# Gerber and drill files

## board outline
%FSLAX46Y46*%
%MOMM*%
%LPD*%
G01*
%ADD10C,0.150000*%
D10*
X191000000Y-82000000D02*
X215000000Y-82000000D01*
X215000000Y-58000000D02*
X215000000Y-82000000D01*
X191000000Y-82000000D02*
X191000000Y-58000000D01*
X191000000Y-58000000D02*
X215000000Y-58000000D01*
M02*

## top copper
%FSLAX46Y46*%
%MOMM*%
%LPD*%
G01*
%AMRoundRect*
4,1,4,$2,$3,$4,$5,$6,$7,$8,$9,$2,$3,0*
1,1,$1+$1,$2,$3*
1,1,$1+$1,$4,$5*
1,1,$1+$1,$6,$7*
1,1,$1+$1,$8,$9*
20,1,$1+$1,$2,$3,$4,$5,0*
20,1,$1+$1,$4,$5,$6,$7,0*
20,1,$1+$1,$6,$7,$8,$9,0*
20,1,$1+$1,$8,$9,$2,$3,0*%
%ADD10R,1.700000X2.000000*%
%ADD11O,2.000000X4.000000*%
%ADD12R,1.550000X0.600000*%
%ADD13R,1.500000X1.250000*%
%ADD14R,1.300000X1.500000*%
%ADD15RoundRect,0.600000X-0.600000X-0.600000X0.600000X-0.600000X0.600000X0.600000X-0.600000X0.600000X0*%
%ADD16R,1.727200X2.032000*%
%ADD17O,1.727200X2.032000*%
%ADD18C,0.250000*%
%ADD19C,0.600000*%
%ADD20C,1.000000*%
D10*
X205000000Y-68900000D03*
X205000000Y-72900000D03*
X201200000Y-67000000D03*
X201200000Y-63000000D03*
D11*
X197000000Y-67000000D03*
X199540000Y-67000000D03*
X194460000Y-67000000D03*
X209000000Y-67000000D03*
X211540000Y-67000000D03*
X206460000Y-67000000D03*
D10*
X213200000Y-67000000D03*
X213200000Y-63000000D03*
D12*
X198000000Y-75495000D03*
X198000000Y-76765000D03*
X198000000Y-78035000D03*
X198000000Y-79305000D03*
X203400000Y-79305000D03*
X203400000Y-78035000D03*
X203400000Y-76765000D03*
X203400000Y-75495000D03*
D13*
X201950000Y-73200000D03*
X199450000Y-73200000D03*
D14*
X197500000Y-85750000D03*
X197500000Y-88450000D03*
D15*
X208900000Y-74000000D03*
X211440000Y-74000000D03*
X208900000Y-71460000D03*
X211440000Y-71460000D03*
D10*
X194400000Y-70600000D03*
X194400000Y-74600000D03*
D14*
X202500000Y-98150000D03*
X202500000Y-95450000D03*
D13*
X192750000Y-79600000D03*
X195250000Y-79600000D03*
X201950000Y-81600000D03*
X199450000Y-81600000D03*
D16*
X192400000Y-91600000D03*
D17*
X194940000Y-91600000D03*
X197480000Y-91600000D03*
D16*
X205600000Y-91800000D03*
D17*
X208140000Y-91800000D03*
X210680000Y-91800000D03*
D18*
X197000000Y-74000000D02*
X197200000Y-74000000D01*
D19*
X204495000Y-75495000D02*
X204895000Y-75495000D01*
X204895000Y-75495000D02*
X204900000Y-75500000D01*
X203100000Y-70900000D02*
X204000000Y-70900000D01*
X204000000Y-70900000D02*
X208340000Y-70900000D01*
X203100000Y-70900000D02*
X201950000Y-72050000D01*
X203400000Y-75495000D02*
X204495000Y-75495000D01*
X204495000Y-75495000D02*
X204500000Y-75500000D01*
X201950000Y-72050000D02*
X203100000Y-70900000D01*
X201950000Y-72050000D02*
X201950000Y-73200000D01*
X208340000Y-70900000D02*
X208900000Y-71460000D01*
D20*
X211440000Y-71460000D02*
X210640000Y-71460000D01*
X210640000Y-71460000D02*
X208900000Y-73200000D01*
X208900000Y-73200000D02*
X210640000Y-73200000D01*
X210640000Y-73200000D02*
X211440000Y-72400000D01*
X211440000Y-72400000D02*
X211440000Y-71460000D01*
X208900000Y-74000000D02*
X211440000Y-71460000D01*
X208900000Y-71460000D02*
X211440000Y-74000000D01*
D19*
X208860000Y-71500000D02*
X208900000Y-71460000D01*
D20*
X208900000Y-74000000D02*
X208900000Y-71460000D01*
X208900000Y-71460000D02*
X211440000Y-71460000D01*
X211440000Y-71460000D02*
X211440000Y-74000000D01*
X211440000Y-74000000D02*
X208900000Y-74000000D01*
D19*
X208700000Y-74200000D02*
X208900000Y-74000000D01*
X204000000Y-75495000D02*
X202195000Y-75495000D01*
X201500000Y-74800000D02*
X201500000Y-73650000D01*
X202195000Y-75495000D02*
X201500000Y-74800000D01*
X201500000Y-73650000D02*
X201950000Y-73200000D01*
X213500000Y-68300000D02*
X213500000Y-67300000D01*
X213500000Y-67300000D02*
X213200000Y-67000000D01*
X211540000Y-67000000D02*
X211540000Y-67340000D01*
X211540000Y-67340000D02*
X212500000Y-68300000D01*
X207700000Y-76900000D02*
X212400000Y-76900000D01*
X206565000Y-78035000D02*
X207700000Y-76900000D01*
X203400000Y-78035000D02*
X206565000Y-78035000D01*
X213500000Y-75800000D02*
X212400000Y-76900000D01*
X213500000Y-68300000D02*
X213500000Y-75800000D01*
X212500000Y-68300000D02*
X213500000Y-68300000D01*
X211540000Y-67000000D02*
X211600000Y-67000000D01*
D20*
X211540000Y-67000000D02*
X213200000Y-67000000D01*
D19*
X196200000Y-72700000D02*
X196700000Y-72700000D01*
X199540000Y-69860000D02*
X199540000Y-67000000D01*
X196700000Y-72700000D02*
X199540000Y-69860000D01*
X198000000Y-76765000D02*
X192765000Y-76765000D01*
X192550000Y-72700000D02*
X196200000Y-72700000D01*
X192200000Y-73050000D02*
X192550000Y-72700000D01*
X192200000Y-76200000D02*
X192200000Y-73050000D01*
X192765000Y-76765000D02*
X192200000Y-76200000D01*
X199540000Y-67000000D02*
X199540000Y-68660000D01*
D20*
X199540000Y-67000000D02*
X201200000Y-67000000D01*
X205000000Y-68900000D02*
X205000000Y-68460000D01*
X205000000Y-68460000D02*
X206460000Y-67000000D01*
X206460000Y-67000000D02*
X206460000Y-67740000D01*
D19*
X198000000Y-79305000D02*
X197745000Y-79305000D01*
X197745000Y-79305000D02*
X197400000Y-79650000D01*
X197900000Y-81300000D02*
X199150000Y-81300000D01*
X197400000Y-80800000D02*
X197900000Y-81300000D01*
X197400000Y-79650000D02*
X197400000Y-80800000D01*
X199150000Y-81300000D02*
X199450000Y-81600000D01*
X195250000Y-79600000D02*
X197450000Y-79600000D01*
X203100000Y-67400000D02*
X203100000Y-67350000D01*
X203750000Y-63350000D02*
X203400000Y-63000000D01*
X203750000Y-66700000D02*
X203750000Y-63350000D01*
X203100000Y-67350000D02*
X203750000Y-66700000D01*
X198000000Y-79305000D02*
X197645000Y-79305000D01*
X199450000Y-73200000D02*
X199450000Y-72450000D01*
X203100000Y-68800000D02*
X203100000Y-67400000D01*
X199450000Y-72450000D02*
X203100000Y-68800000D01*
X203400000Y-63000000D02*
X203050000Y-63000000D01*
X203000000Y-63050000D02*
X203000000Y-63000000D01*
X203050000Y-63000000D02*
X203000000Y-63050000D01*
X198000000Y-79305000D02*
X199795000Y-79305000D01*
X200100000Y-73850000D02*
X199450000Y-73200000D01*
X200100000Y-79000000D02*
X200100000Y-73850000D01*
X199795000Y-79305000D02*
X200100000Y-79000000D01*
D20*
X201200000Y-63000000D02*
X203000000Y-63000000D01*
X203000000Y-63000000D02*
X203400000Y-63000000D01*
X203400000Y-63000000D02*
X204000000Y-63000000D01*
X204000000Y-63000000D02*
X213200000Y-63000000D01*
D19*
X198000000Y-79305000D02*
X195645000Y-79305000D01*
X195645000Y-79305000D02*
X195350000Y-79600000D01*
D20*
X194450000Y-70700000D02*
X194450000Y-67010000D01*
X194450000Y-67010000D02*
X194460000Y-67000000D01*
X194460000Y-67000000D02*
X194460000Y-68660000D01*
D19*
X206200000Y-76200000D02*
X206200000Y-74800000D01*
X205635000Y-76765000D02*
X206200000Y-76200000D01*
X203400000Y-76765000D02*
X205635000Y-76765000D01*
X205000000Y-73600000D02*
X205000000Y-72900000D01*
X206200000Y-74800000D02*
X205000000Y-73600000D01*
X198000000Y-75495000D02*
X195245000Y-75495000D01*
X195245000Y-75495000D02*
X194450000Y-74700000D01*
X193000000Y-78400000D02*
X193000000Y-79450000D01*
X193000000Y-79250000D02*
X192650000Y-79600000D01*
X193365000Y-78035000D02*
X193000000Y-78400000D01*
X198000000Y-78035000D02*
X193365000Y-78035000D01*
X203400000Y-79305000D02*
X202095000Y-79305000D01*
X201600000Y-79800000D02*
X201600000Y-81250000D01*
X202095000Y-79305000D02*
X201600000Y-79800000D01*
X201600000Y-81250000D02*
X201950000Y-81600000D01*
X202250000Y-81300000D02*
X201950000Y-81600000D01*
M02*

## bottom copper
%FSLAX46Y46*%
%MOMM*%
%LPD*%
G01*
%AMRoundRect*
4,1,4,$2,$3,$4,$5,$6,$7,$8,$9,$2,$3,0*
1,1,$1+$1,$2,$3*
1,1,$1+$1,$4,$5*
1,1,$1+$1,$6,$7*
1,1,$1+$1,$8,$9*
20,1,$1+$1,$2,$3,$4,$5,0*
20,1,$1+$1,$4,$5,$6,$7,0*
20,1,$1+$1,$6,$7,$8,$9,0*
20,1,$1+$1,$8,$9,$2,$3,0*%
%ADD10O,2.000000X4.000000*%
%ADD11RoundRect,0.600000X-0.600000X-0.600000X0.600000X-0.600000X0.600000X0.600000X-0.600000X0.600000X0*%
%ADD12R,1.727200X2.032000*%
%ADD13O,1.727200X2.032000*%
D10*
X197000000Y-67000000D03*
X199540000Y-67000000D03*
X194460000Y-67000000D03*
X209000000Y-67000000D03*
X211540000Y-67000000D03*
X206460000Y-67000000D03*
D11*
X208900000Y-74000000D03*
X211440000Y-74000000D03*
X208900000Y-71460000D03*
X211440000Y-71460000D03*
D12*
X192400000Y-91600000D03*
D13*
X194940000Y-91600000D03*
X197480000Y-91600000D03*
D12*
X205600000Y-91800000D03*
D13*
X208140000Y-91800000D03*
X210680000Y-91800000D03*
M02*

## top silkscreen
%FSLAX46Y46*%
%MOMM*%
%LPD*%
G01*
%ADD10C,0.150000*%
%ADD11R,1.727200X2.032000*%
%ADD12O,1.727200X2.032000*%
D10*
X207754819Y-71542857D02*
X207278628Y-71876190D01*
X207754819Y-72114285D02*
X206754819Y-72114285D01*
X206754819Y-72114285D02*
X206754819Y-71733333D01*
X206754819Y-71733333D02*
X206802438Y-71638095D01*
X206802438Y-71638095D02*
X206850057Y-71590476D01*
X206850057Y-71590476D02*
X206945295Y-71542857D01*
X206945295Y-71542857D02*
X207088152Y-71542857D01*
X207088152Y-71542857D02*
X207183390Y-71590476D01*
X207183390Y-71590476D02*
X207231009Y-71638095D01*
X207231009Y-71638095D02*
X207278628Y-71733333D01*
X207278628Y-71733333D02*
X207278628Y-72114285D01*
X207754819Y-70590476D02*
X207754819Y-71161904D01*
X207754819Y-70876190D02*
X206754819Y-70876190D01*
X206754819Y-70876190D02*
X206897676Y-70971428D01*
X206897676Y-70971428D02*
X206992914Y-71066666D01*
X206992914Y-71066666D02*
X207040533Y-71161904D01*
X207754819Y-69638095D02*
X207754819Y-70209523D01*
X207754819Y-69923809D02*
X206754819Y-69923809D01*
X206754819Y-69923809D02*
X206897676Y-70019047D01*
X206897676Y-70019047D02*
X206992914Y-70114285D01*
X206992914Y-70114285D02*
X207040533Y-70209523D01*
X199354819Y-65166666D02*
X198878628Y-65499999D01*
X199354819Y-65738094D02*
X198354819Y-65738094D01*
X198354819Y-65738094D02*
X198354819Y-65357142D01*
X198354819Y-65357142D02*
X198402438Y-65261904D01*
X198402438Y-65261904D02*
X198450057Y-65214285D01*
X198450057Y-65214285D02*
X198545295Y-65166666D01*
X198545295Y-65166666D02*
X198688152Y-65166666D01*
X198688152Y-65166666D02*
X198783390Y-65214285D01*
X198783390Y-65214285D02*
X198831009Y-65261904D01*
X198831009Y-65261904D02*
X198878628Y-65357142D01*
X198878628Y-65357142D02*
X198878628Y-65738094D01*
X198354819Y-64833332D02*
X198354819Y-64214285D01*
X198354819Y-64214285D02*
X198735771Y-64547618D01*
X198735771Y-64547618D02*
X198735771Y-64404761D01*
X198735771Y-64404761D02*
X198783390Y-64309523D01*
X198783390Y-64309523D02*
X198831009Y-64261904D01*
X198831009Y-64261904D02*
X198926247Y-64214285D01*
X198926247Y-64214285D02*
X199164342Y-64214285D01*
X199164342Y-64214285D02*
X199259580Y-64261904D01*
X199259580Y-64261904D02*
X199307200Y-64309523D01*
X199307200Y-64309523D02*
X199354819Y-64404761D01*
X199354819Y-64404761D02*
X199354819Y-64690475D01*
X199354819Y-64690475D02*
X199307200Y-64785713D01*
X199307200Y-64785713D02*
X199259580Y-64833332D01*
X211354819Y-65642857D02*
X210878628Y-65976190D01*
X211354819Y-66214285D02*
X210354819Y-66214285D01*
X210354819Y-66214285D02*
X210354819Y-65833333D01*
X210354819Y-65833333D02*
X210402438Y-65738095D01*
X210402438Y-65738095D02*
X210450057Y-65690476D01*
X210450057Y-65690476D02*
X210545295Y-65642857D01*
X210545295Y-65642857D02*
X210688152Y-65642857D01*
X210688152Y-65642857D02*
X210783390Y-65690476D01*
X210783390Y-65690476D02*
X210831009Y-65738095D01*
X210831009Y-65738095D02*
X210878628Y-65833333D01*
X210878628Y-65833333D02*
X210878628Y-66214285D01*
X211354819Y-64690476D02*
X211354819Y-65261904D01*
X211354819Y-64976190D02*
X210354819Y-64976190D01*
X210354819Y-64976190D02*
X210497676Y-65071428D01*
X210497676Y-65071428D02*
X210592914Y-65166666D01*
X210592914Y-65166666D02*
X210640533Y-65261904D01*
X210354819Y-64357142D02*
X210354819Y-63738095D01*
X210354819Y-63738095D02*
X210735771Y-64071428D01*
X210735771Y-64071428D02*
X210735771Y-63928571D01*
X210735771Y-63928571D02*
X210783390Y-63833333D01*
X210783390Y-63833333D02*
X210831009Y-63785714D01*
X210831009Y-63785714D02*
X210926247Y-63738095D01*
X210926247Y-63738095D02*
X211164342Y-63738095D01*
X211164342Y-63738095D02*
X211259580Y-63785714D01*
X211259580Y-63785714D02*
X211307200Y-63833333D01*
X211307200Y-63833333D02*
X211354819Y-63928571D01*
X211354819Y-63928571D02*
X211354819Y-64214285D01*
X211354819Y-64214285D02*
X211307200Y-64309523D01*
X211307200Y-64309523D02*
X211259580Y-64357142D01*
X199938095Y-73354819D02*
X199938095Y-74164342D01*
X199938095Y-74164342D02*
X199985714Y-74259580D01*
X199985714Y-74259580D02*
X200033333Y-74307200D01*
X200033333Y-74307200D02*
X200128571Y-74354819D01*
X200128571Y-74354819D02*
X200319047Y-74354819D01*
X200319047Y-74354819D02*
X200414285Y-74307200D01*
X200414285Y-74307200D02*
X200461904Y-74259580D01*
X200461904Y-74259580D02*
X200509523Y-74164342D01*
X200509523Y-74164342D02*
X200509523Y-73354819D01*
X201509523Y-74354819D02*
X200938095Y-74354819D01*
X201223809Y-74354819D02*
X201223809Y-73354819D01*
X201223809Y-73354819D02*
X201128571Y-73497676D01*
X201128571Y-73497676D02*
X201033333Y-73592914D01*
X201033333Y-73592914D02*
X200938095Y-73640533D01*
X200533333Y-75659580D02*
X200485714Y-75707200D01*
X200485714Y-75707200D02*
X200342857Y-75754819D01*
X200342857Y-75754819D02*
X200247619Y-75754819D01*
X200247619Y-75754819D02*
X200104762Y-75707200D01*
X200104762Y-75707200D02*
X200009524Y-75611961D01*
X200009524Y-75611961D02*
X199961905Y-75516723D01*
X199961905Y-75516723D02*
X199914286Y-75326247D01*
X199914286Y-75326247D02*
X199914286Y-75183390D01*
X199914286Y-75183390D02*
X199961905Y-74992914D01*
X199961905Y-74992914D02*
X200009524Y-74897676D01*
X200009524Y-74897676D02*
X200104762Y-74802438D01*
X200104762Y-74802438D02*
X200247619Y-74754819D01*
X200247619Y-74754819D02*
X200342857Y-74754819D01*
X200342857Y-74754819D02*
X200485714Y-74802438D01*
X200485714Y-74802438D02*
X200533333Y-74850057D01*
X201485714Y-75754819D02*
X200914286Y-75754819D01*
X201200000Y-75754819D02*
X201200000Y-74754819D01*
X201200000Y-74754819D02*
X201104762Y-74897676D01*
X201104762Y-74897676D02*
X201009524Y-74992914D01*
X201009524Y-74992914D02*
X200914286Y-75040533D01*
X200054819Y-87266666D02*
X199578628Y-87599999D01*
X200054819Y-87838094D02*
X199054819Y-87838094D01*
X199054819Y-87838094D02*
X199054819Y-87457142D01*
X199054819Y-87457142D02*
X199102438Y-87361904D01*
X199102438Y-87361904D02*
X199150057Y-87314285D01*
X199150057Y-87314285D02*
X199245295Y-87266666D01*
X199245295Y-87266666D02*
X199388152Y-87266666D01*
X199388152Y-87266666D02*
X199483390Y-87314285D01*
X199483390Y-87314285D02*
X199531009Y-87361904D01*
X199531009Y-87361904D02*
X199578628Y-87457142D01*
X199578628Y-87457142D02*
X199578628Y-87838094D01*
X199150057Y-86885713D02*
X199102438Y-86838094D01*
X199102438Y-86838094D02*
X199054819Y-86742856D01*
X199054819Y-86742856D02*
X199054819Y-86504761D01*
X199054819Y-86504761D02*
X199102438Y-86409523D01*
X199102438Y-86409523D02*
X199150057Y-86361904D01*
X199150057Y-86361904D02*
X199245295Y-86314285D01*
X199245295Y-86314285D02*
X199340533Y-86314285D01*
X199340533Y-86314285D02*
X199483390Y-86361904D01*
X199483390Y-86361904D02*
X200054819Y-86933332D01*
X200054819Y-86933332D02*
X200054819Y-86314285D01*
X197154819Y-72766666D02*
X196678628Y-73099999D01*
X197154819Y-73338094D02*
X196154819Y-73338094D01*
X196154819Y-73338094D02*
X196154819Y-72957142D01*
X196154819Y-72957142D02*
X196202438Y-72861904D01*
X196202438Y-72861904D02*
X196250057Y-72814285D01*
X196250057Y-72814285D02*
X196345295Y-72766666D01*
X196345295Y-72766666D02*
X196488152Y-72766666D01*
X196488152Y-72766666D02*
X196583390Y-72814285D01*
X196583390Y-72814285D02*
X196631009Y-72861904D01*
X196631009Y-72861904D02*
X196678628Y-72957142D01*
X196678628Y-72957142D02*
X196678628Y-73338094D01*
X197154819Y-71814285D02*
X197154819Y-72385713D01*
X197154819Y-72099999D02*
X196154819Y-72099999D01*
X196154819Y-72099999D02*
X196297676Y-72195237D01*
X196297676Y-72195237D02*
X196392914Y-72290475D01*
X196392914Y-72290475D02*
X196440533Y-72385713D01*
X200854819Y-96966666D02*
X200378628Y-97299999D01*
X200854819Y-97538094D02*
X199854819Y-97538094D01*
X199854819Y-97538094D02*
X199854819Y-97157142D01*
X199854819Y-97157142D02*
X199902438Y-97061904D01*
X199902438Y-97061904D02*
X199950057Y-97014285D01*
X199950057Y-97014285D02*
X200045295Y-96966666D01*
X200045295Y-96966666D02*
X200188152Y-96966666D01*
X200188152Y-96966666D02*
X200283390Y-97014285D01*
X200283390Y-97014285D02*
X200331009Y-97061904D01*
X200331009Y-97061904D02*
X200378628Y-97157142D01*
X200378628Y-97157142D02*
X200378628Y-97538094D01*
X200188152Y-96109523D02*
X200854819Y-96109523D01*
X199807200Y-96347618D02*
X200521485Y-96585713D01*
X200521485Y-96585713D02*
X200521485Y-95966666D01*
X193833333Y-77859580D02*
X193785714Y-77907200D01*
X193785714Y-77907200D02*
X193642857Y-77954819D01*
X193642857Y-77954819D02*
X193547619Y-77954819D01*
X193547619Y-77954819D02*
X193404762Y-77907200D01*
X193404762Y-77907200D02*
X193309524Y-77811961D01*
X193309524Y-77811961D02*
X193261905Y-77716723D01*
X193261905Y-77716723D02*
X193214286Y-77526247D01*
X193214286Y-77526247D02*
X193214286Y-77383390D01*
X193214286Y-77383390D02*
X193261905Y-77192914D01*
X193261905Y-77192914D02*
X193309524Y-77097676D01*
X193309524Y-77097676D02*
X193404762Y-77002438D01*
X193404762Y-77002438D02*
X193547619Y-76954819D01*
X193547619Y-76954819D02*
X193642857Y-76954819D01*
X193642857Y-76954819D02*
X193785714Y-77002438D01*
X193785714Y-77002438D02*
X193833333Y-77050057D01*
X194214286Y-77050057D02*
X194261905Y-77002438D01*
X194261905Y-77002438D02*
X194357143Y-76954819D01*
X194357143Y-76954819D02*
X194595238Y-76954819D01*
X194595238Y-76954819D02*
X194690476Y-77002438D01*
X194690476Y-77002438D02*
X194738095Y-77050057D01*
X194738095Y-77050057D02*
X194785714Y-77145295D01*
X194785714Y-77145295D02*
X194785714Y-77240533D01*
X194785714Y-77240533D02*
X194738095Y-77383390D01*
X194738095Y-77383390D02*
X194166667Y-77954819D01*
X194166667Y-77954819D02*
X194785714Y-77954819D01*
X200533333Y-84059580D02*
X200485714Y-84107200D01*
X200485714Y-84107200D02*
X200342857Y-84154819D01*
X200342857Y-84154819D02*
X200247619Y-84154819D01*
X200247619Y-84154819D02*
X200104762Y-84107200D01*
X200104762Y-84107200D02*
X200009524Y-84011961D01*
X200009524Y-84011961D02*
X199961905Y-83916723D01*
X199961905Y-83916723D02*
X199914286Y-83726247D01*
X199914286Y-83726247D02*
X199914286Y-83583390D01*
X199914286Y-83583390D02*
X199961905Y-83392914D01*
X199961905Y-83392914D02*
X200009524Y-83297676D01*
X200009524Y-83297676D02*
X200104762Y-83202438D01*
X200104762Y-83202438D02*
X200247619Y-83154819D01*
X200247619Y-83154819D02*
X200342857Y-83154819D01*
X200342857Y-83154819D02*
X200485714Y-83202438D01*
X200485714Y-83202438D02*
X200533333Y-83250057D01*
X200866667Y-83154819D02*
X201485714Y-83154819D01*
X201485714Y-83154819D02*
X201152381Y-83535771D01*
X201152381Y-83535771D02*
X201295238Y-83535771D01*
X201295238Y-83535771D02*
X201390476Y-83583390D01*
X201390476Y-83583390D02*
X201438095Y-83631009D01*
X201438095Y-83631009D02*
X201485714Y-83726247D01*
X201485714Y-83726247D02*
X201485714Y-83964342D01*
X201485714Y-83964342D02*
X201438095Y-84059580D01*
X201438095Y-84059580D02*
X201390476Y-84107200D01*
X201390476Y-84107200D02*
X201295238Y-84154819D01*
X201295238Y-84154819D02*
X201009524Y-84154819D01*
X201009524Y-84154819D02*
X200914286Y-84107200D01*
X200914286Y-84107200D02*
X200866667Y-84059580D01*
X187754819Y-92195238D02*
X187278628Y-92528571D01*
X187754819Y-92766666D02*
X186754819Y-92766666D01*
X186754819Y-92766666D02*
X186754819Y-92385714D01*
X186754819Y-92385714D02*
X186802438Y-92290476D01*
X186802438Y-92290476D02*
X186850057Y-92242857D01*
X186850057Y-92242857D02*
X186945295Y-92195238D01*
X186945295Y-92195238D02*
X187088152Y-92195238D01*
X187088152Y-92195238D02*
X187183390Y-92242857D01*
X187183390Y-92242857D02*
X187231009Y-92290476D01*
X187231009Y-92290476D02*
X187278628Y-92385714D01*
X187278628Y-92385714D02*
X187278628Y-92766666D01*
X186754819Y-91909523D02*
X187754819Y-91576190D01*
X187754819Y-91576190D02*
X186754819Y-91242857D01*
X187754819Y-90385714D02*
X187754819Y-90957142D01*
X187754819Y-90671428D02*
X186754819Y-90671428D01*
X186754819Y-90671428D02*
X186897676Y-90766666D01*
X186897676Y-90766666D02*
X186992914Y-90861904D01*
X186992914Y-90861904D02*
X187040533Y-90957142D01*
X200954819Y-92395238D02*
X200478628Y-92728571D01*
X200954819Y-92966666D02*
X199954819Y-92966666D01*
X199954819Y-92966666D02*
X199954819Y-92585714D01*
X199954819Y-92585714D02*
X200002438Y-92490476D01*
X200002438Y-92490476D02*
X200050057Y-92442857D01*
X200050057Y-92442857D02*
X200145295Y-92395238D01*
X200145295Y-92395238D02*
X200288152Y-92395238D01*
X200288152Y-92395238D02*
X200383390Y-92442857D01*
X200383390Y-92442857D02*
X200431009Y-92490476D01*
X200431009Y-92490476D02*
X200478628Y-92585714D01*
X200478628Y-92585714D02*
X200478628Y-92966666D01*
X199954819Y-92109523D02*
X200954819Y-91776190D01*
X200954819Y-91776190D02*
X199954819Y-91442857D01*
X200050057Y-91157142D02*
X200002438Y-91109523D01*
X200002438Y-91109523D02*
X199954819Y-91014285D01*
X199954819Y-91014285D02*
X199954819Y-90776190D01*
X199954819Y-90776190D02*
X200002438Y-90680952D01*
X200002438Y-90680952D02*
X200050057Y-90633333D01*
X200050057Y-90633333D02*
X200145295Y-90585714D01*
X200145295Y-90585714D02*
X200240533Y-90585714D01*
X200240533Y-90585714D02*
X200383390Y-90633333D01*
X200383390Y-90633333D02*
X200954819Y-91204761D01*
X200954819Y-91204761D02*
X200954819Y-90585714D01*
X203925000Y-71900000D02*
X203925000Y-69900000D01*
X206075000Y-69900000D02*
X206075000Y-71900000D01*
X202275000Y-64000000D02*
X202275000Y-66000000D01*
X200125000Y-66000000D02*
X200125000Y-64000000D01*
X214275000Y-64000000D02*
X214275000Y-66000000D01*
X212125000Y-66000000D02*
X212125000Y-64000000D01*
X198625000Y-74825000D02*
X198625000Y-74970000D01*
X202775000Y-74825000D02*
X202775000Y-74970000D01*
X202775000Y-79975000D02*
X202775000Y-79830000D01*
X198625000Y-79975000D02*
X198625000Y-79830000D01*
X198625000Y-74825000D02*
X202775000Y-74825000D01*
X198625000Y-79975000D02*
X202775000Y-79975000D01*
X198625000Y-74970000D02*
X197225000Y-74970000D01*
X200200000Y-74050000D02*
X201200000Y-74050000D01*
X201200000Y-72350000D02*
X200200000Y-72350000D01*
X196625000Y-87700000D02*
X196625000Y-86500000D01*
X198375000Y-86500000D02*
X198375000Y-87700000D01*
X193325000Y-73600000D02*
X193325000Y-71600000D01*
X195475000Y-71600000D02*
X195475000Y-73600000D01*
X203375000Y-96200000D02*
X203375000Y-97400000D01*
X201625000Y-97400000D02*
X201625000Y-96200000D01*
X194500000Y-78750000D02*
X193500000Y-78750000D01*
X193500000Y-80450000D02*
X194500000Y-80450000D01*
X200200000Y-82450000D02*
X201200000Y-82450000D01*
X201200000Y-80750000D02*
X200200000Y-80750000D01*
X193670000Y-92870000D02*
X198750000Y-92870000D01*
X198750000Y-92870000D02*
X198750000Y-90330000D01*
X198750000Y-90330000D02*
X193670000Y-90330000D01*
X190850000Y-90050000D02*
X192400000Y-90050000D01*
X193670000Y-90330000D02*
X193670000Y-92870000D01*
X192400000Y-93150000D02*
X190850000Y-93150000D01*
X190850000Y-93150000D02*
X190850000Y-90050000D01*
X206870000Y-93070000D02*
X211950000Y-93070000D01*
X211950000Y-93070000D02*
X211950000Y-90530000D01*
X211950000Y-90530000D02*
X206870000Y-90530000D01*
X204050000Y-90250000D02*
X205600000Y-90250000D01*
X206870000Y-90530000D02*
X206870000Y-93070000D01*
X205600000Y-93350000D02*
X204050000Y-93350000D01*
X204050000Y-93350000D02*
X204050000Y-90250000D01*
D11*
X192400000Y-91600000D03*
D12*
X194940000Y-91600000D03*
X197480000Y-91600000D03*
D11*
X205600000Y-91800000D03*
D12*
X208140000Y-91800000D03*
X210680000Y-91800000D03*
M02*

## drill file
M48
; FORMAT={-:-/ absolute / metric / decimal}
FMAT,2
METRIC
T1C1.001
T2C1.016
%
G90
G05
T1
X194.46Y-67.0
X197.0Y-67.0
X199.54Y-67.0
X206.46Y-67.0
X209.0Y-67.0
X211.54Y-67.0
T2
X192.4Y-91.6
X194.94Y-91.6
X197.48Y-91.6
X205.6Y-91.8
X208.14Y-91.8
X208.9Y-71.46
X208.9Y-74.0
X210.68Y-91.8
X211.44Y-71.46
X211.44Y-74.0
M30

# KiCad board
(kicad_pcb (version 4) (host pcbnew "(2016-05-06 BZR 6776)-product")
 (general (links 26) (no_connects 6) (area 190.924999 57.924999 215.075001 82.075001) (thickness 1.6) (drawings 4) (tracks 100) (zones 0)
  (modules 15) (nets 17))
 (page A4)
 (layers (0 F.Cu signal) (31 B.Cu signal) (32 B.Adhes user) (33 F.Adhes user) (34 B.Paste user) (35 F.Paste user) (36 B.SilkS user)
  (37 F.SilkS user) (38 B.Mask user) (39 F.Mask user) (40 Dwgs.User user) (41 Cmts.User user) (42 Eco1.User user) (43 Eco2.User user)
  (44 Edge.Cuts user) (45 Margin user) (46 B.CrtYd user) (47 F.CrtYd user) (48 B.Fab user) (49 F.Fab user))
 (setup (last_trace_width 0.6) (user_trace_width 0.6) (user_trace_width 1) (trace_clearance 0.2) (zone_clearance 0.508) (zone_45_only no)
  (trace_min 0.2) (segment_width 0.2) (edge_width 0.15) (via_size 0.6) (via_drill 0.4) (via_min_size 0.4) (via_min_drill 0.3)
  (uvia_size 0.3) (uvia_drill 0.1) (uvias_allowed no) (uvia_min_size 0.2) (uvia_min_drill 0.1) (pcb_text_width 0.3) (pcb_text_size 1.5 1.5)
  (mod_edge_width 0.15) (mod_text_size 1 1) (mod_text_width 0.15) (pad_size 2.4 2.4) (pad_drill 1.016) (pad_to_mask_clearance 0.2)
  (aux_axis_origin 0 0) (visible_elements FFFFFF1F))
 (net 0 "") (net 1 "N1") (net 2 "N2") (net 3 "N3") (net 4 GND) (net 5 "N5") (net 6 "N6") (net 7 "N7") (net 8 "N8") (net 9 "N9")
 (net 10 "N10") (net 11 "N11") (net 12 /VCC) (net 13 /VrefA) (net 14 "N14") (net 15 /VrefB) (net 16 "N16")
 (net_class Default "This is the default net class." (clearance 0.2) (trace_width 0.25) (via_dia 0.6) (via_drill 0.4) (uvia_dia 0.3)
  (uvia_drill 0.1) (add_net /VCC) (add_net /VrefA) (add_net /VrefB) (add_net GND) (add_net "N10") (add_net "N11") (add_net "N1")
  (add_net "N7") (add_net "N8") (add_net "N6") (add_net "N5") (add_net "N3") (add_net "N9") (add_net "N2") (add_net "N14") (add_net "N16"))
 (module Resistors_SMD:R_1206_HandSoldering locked (layer F.Cu) (at 205 70.9 270)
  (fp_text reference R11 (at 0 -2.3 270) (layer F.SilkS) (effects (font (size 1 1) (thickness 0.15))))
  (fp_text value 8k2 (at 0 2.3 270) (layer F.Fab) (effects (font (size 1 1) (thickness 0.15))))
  (fp_line (start 1 1.075) (end -1 1.075) (layer F.SilkS) (width 0.15))
  (fp_line (start -1 -1.075) (end 1 -1.075) (layer F.SilkS) (width 0.15))
  (pad 1 smd rect (at -2 0 270) (size 2 1.7) (layers F.Cu F.Paste F.Mask) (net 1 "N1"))
  (pad 2 smd rect (at 2 0 270) (size 2 1.7) (layers F.Cu F.Paste F.Mask) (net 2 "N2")))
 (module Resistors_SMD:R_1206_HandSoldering (layer F.Cu) (at 201.2 65 90)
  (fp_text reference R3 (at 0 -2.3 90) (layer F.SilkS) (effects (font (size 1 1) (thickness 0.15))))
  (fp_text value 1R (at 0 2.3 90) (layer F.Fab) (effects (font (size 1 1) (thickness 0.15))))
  (fp_line (start 1 1.075) (end -1 1.075) (layer F.SilkS) (width 0.15))
  (fp_line (start -1 -1.075) (end 1 -1.075) (layer F.SilkS) (width 0.15))
  (pad 1 smd rect (at -2 0 90) (size 2 1.7) (layers F.Cu F.Paste F.Mask) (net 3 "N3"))
  (pad 2 smd rect (at 2 0 90) (size 2 1.7) (layers F.Cu F.Paste F.Mask) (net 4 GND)))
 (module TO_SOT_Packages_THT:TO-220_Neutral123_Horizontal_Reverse (layer B.Cu) (at 197 67 180)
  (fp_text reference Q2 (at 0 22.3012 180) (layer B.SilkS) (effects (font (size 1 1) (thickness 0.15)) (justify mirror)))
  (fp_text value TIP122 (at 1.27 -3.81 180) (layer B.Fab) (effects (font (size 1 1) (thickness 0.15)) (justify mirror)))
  (pad 2 thru_hole oval (at 0 0 90) (size 4 2) (drill 1.00076) (layers *.Cu *.Mask B.SilkS) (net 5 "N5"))
  (pad 3 thru_hole oval (at -2.54 0 90) (size 4 2) (drill 1.00076) (layers *.Cu *.Mask B.SilkS) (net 3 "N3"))
  (pad 1 thru_hole oval (at 2.54 0 90) (size 4 2) (drill 1.00076) (layers *.Cu *.Mask B.SilkS) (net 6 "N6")))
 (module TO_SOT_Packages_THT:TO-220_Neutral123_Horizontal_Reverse (layer B.Cu) (at 209 67 180)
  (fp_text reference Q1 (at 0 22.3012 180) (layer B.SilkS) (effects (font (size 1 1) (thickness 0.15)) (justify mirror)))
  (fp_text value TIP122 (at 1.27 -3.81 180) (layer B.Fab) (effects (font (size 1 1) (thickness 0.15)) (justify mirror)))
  (pad 2 thru_hole oval (at 0 0 90) (size 4 2) (drill 1.00076) (layers *.Cu *.Mask B.SilkS) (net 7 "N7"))
  (pad 3 thru_hole oval (at -2.54 0 90) (size 4 2) (drill 1.00076) (layers *.Cu *.Mask B.SilkS) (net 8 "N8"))
  (pad 1 thru_hole oval (at 2.54 0 90) (size 4 2) (drill 1.00076) (layers *.Cu *.Mask B.SilkS) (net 1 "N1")))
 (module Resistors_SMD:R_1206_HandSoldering (layer F.Cu) (at 213.2 65 90)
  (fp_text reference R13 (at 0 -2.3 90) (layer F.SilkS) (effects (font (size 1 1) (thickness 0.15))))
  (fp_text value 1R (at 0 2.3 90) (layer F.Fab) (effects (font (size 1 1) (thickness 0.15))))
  (fp_line (start 1 1.075) (end -1 1.075) (layer F.SilkS) (width 0.15))
  (fp_line (start -1 -1.075) (end 1 -1.075) (layer F.SilkS) (width 0.15))
  (pad 1 smd rect (at -2 0 90) (size 2 1.7) (layers F.Cu F.Paste F.Mask) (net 8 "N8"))
  (pad 2 smd rect (at 2 0 90) (size 2 1.7) (layers F.Cu F.Paste F.Mask) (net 4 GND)))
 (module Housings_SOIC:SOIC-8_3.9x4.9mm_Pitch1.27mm (layer F.Cu) (at 200.7 77.4)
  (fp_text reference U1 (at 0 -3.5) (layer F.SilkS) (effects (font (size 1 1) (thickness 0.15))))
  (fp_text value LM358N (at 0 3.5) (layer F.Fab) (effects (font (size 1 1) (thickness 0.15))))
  (fp_line (start -2.075 -2.575) (end -2.075 -2.43) (layer F.SilkS) (width 0.15))
  (fp_line (start 2.075 -2.575) (end 2.075 -2.43) (layer F.SilkS) (width 0.15))
  (fp_line (start 2.075 2.575) (end 2.075 2.43) (layer F.SilkS) (width 0.15))
  (fp_line (start -2.075 2.575) (end -2.075 2.43) (layer F.SilkS) (width 0.15))
  (fp_line (start -2.075 -2.575) (end 2.075 -2.575) (layer F.SilkS) (width 0.15))
  (fp_line (start -2.075 2.575) (end 2.075 2.575) (layer F.SilkS) (width 0.15))
  (fp_line (start -2.075 -2.43) (end -3.475 -2.43) (layer F.SilkS) (width 0.15))
  (pad 1 smd rect (at -2.7 -1.905) (size 1.55 0.6) (layers F.Cu F.Paste F.Mask) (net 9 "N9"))
  (pad 2 smd rect (at -2.7 -0.635) (size 1.55 0.6) (layers F.Cu F.Paste F.Mask) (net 3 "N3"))
  (pad 3 smd rect (at -2.7 0.635) (size 1.55 0.6) (layers F.Cu F.Paste F.Mask) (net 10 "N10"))
  (pad 4 smd rect (at -2.7 1.905) (size 1.55 0.6) (layers F.Cu F.Paste F.Mask) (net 4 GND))
  (pad 5 smd rect (at 2.7 1.905) (size 1.55 0.6) (layers F.Cu F.Paste F.Mask) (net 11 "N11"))
  (pad 6 smd rect (at 2.7 0.635) (size 1.55 0.6) (layers F.Cu F.Paste F.Mask) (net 8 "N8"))
  (pad 7 smd rect (at 2.7 -0.635) (size 1.55 0.6) (layers F.Cu F.Paste F.Mask) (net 2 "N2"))
  (pad 8 smd rect (at 2.7 -1.905) (size 1.55 0.6) (layers F.Cu F.Paste F.Mask) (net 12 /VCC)))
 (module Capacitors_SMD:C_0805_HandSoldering (layer F.Cu) (at 200.7 73.2 180)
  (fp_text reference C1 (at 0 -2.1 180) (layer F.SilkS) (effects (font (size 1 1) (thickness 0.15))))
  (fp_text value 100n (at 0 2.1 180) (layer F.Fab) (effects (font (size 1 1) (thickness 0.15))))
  (fp_line (start 0.5 -0.85) (end -0.5 -0.85) (layer F.SilkS) (width 0.15))
  (fp_line (start -0.5 0.85) (end 0.5 0.85) (layer F.SilkS) (width 0.15))
  (pad 1 smd rect (at -1.25 0 180) (size 1.5 1.25) (layers F.Cu F.Paste F.Mask) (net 12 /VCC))
  (pad 2 smd rect (at 1.25 0 180) (size 1.5 1.25) (layers F.Cu F.Paste F.Mask) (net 4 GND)))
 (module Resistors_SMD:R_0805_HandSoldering (layer F.Cu) (at 197.5 87.1 270)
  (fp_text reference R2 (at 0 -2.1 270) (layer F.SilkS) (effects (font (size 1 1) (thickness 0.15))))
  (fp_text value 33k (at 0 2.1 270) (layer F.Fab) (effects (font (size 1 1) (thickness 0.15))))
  (fp_line (start 0.6 0.875) (end -0.6 0.875) (layer F.SilkS) (width 0.15))
  (fp_line (start -0.6 -0.875) (end 0.6 -0.875) (layer F.SilkS) (width 0.15))
  (pad 1 smd rect (at -1.35 0 270) (size 1.5 1.3) (layers F.Cu F.Paste F.Mask) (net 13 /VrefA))
  (pad 2 smd rect (at 1.35 0 270) (size 1.5 1.3) (layers F.Cu F.Paste F.Mask) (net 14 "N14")))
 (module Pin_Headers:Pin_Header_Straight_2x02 (layer B.Cu) (at 208.9 74)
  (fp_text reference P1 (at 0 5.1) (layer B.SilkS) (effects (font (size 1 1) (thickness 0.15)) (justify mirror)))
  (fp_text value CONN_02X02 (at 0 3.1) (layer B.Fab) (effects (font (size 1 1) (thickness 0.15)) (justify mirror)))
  (pad 1 thru_hole roundrect (at 0 0) (size 2.4 2.4) (drill 1.016) (layers *.Cu *.Mask B.SilkS) (roundrect_rratio 0.25) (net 12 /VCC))
  (pad 2 thru_hole roundrect (at 2.54 0) (size 2.4 2.4) (drill 1.016) (layers *.Cu *.Mask B.SilkS) (roundrect_rratio 0.25) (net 12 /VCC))
  (pad 3 thru_hole roundrect (at 0 -2.54) (size 2.4 2.4) (drill 1.016) (layers *.Cu *.Mask B.SilkS) (roundrect_rratio 0.25) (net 12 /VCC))
  (pad 4 thru_hole roundrect (at 2.54 -2.54) (size 2.4 2.4) (drill 1.016) (layers *.Cu *.Mask B.SilkS) (roundrect_rratio 0.25) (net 12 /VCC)))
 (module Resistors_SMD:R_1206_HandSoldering (layer F.Cu) (at 194.4 72.6 270)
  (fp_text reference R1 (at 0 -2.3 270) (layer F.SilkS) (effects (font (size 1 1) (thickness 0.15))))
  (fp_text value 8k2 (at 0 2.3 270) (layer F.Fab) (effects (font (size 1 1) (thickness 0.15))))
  (fp_line (start 1 1.075) (end -1 1.075) (layer F.SilkS) (width 0.15))
  (fp_line (start -1 -1.075) (end 1 -1.075) (layer F.SilkS) (width 0.15))
  (pad 1 smd rect (at -2 0 270) (size 2 1.7) (layers F.Cu F.Paste F.Mask) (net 6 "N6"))
  (pad 2 smd rect (at 2 0 270) (size 2 1.7) (layers F.Cu F.Paste F.Mask) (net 9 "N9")))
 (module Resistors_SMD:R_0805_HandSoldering (layer F.Cu) (at 202.5 96.8 90)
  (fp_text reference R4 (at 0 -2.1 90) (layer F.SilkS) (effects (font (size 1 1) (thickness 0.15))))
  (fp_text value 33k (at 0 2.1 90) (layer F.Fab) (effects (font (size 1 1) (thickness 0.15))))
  (fp_line (start 0.6 0.875) (end -0.6 0.875) (layer F.SilkS) (width 0.15))
  (fp_line (start -0.6 -0.875) (end 0.6 -0.875) (layer F.SilkS) (width 0.15))
  (pad 1 smd rect (at -1.35 0 90) (size 1.5 1.3) (layers F.Cu F.Paste F.Mask) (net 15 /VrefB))
  (pad 2 smd rect (at 1.35 0 90) (size 1.5 1.3) (layers F.Cu F.Paste F.Mask) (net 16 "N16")))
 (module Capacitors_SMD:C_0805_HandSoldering (layer F.Cu) (at 194 79.6)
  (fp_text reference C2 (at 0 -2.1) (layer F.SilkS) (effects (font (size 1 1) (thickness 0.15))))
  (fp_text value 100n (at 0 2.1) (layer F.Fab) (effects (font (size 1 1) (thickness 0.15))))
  (fp_line (start 0.5 -0.85) (end -0.5 -0.85) (layer F.SilkS) (width 0.15))
  (fp_line (start -0.5 0.85) (end 0.5 0.85) (layer F.SilkS) (width 0.15))
  (pad 1 smd rect (at -1.25 0) (size 1.5 1.25) (layers F.Cu F.Paste F.Mask) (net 10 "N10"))
  (pad 2 smd rect (at 1.25 0) (size 1.5 1.25) (layers F.Cu F.Paste F.Mask) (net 4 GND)))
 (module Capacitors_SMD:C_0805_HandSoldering (layer F.Cu) (at 200.7 81.6 180)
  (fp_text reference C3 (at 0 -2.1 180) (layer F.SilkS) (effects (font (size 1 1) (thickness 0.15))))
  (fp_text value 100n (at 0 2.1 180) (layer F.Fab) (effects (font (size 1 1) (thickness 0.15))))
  (fp_line (start 0.5 -0.85) (end -0.5 -0.85) (layer F.SilkS) (width 0.15))
  (fp_line (start -0.5 0.85) (end 0.5 0.85) (layer F.SilkS) (width 0.15))
  (pad 1 smd rect (at -1.25 0 180) (size 1.5 1.25) (layers F.Cu F.Paste F.Mask) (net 11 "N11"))
  (pad 2 smd rect (at 1.25 0 180) (size 1.5 1.25) (layers F.Cu F.Paste F.Mask) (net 4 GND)))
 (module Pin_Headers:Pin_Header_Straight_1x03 (layer F.Cu) (at 192.4 91.6 90)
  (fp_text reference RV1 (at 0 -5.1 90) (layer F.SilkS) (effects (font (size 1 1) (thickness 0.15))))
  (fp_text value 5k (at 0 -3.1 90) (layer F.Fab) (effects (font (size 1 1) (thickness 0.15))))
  (fp_line (start -1.27 1.27) (end -1.27 6.35) (layer F.SilkS) (width 0.15))
  (fp_line (start -1.27 6.35) (end 1.27 6.35) (layer F.SilkS) (width 0.15))
  (fp_line (start 1.27 6.35) (end 1.27 1.27) (layer F.SilkS) (width 0.15))
  (fp_line (start 1.55 -1.55) (end 1.55 0) (layer F.SilkS) (width 0.15))
  (fp_line (start 1.27 1.27) (end -1.27 1.27) (layer F.SilkS) (width 0.15))
  (fp_line (start -1.55 0) (end -1.55 -1.55) (layer F.SilkS) (width 0.15))
  (fp_line (start -1.55 -1.55) (end 1.55 -1.55) (layer F.SilkS) (width 0.15))
  (pad 1 thru_hole rect (at 0 0 90) (size 2.032 1.7272) (drill 1.016) (layers *.Cu *.Mask F.SilkS) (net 4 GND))
  (pad 2 thru_hole oval (at 0 2.54 90) (size 2.032 1.7272) (drill 1.016) (layers *.Cu *.Mask F.SilkS) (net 10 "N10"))
  (pad 3 thru_hole oval (at 0 5.08 90) (size 2.032 1.7272) (drill 1.016) (layers *.Cu *.Mask F.SilkS) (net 14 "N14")))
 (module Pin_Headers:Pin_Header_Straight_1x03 (layer F.Cu) (at 205.6 91.8 90)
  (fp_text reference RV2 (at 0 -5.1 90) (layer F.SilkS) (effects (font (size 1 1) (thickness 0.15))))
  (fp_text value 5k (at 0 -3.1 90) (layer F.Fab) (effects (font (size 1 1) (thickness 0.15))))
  (fp_line (start -1.27 1.27) (end -1.27 6.35) (layer F.SilkS) (width 0.15))
  (fp_line (start -1.27 6.35) (end 1.27 6.35) (layer F.SilkS) (width 0.15))
  (fp_line (start 1.27 6.35) (end 1.27 1.27) (layer F.SilkS) (width 0.15))
  (fp_line (start 1.55 -1.55) (end 1.55 0) (layer F.SilkS) (width 0.15))
  (fp_line (start 1.27 1.27) (end -1.27 1.27) (layer F.SilkS) (width 0.15))
  (fp_line (start -1.55 0) (end -1.55 -1.55) (layer F.SilkS) (width 0.15))
  (fp_line (start -1.55 -1.55) (end 1.55 -1.55) (layer F.SilkS) (width 0.15))
  (pad 1 thru_hole rect (at 0 0 90) (size 2.032 1.7272) (drill 1.016) (layers *.Cu *.Mask F.SilkS) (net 4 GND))
  (pad 2 thru_hole oval (at 0 2.54 90) (size 2.032 1.7272) (drill 1.016) (layers *.Cu *.Mask F.SilkS) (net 11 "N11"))
  (pad 3 thru_hole oval (at 0 5.08 90) (size 2.032 1.7272) (drill 1.016) (layers *.Cu *.Mask F.SilkS) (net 16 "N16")))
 (gr_line (start 191 82) (end 215 82) (angle 90) (layer Edge.Cuts) (width 0.15))
 (gr_line (start 215 58) (end 215 82) (angle 90) (layer Edge.Cuts) (width 0.15))
 (gr_line (start 191 82) (end 191 58) (angle 90) (layer Edge.Cuts) (width 0.15))
 (gr_line (start 191 58) (end 215 58) (angle 90) (layer Edge.Cuts) (width 0.15))
 (segment (start 197 74) (end 197.2 74) (width 0.25) (layer F.Cu) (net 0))
 (segment (start 204.495 75.495) (end 204.895 75.495) (width 0.6) (layer F.Cu) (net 12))
 (segment (start 204.895 75.495) (end 204.9 75.5) (width 0.6) (layer F.Cu) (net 12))
 (segment (start 203.1 70.9) (end 204 70.9) (width 0.6) (layer F.Cu) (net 12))
 (segment (start 204 70.9) (end 208.34 70.9) (width 0.6) (layer F.Cu) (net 12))
 (segment (start 203.1 70.9) (end 201.95 72.05) (width 0.6) (layer F.Cu) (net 12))
 (segment (start 203.4 75.495) (end 204.495 75.495) (width 0.6) (layer F.Cu) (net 12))
 (segment (start 204.495 75.495) (end 204.5 75.5) (width 0.6) (layer F.Cu) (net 12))
 (segment (start 201.95 72.05) (end 203.1 70.9) (width 0.6) (layer F.Cu) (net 12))
 (segment (start 201.95 72.05) (end 201.95 73.2) (width 0.6) (layer F.Cu) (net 12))
 (segment (start 208.34 70.9) (end 208.9 71.46) (width 0.6) (layer F.Cu) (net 12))
 (segment (start 211.44 71.46) (end 210.64 71.46) (width 1) (layer F.Cu) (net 12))
 (segment (start 210.64 71.46) (end 208.9 73.2) (width 1) (layer F.Cu) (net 12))
 (segment (start 208.9 73.2) (end 210.64 73.2) (width 1) (layer F.Cu) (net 12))
 (segment (start 210.64 73.2) (end 211.44 72.4) (width 1) (layer F.Cu) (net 12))
 (segment (start 211.44 72.4) (end 211.44 71.46) (width 1) (layer F.Cu) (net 12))
 (segment (start 208.9 74) (end 211.44 71.46) (width 1) (layer F.Cu) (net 12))
 (segment (start 208.9 71.46) (end 211.44 74) (width 1) (layer F.Cu) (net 12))
 (segment (start 208.86 71.5) (end 208.9 71.46) (width 0.6) (layer F.Cu) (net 12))
 (segment (start 208.9 74) (end 208.9 71.46) (width 1) (layer F.Cu) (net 12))
 (segment (start 208.9 71.46) (end 211.44 71.46) (width 1) (layer F.Cu) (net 12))
 (segment (start 211.44 71.46) (end 211.44 74) (width 1) (layer F.Cu) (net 12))
 (segment (start 211.44 74) (end 208.9 74) (width 1) (layer F.Cu) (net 12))
 (segment (start 208.7 74.2) (end 208.9 74) (width 0.6) (layer F.Cu) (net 12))
 (segment (start 204 75.495) (end 202.195 75.495) (width 0.6) (layer F.Cu) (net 12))
 (segment (start 201.5 74.8) (end 201.5 73.65) (width 0.6) (layer F.Cu) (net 12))
 (segment (start 202.195 75.495) (end 201.5 74.8) (width 0.6) (layer F.Cu) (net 12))
 (segment (start 201.5 73.65) (end 201.95 73.2) (width 0.6) (layer F.Cu) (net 12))
 (segment (start 213.5 68.3) (end 213.5 67.3) (width 0.6) (layer F.Cu) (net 8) (status 800000))
 (segment (start 213.5 67.3) (end 213.2 67) (width 0.6) (layer F.Cu) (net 8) (status C00000))
 (segment (start 211.54 67) (end 211.54 67.34) (width 0.6) (layer F.Cu) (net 8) (status C00000))
 (segment (start 211.54 67.34) (end 212.5 68.3) (width 0.6) (layer F.Cu) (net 8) (status 400000))
 (segment (start 207.7 76.9) (end 212.4 76.9) (width 0.6) (layer F.Cu) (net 8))
 (segment (start 206.565 78.035) (end 207.7 76.9) (width 0.6) (layer F.Cu) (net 8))
 (segment (start 203.4 78.035) (end 206.565 78.035) (width 0.6) (layer F.Cu) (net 8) (status 400000))
 (segment (start 213.5 75.8) (end 212.4 76.9) (width 0.6) (layer F.Cu) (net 8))
 (segment (start 213.5 68.3) (end 213.5 75.8) (width 0.6) (layer F.Cu) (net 8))
 (segment (start 212.5 68.3) (end 213.5 68.3) (width 0.6) (layer F.Cu) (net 8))
 (segment (start 211.54 67) (end 211.6 67) (width 0.6) (layer F.Cu) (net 8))
 (segment (start 211.54 67) (end 213.2 67) (width 1) (layer F.Cu) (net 8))
 (segment (start 196.2 72.7) (end 196.7 72.7) (width 0.6) (layer F.Cu) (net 3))
 (segment (start 199.54 69.86) (end 199.54 67) (width 0.6) (layer F.Cu) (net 3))
 (segment (start 196.7 72.7) (end 199.54 69.86) (width 0.6) (layer F.Cu) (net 3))
 (segment (start 198 76.765) (end 192.765 76.765) (width 0.6) (layer F.Cu) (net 3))
 (segment (start 192.55 72.7) (end 196.2 72.7) (width 0.6) (layer F.Cu) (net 3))
 (segment (start 192.2 73.05) (end 192.55 72.7) (width 0.6) (layer F.Cu) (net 3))
 (segment (start 192.2 76.2) (end 192.2 73.05) (width 0.6) (layer F.Cu) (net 3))
 (segment (start 192.765 76.765) (end 192.2 76.2) (width 0.6) (layer F.Cu) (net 3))
 (segment (start 199.54 67) (end 199.54 68.66) (width 0.6) (layer F.Cu) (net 3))
 (segment (start 199.54 67) (end 201.2 67) (width 1) (layer F.Cu) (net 3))
 (segment (start 205 68.9) (end 205 68.46) (width 1) (layer F.Cu) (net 1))
 (segment (start 205 68.46) (end 206.46 67) (width 1) (layer F.Cu) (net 1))
 (segment (start 206.46 67) (end 206.46 67.74) (width 1) (layer F.Cu) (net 1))
 (segment (start 198 79.305) (end 197.745 79.305) (width 0.6) (layer F.Cu) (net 4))
 (segment (start 197.745 79.305) (end 197.4 79.65) (width 0.6) (layer F.Cu) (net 4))
 (segment (start 197.9 81.3) (end 199.15 81.3) (width 0.6) (layer F.Cu) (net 4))
 (segment (start 197.4 80.8) (end 197.9 81.3) (width 0.6) (layer F.Cu) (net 4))
 (segment (start 197.4 79.65) (end 197.4 80.8) (width 0.6) (layer F.Cu) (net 4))
 (segment (start 199.15 81.3) (end 199.45 81.6) (width 0.6) (layer F.Cu) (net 4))
 (segment (start 195.25 79.6) (end 197.45 79.6) (width 0.6) (layer F.Cu) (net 4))
 (segment (start 203.1 67.4) (end 203.1 67.35) (width 0.6) (layer F.Cu) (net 4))
 (segment (start 203.75 63.35) (end 203.4 63) (width 0.6) (layer F.Cu) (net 4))
 (segment (start 203.75 66.7) (end 203.75 63.35) (width 0.6) (layer F.Cu) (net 4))
 (segment (start 203.1 67.35) (end 203.75 66.7) (width 0.6) (layer F.Cu) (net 4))
 (segment (start 198 79.305) (end 197.645 79.305) (width 0.6) (layer F.Cu) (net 4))
 (segment (start 199.45 73.2) (end 199.45 72.45) (width 0.6) (layer F.Cu) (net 4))
 (segment (start 203.1 68.8) (end 203.1 67.4) (width 0.6) (layer F.Cu) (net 4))
 (segment (start 199.45 72.45) (end 203.1 68.8) (width 0.6) (layer F.Cu) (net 4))
 (segment (start 203.4 63) (end 203.05 63) (width 0.6) (layer F.Cu) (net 4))
 (segment (start 203 63.05) (end 203 63) (width 0.6) (layer F.Cu) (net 4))
 (segment (start 203.05 63) (end 203 63.05) (width 0.6) (layer F.Cu) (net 4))
 (segment (start 198 79.305) (end 199.795 79.305) (width 0.6) (layer F.Cu) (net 4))
 (segment (start 200.1 73.85) (end 199.45 73.2) (width 0.6) (layer F.Cu) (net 4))
 (segment (start 200.1 79) (end 200.1 73.85) (width 0.6) (layer F.Cu) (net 4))
 (segment (start 199.795 79.305) (end 200.1 79) (width 0.6) (layer F.Cu) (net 4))
 (segment (start 201.2 63) (end 203 63) (width 1) (layer F.Cu) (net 4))
 (segment (start 203 63) (end 203.4 63) (width 1) (layer F.Cu) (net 4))
 (segment (start 203.4 63) (end 204 63) (width 1) (layer F.Cu) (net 4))
 (segment (start 204 63) (end 213.2 63) (width 1) (layer F.Cu) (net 4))
 (segment (start 198 79.305) (end 195.645 79.305) (width 0.6) (layer F.Cu) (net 4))
 (segment (start 195.645 79.305) (end 195.35 79.6) (width 0.6) (layer F.Cu) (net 4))
 (segment (start 194.45 70.7) (end 194.45 67.01) (width 1) (layer F.Cu) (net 6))
 (segment (start 194.45 67.01) (end 194.46 67) (width 1) (layer F.Cu) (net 6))
 (segment (start 194.46 67) (end 194.46 68.66) (width 1) (layer F.Cu) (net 6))
 (segment (start 206.2 76.2) (end 206.2 74.8) (width 0.6) (layer F.Cu) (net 2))
 (segment (start 205.635 76.765) (end 206.2 76.2) (width 0.6) (layer F.Cu) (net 2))
 (segment (start 203.4 76.765) (end 205.635 76.765) (width 0.6) (layer F.Cu) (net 2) (status 400000))
 (segment (start 205 73.6) (end 205 72.9) (width 0.6) (layer F.Cu) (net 2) (status 800000))
 (segment (start 206.2 74.8) (end 205 73.6) (width 0.6) (layer F.Cu) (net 2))
 (segment (start 198 75.495) (end 195.245 75.495) (width 0.6) (layer F.Cu) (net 9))
 (segment (start 195.245 75.495) (end 194.45 74.7) (width 0.6) (layer F.Cu) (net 9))
 (segment (start 193 78.4) (end 193 79.45) (width 0.6) (layer F.Cu) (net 10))
 (segment (start 193 79.25) (end 192.65 79.6) (width 0.6) (layer F.Cu) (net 10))
 (segment (start 193.365 78.035) (end 193 78.4) (width 0.6) (layer F.Cu) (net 10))
 (segment (start 198 78.035) (end 193.365 78.035) (width 0.6) (layer F.Cu) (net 10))
 (segment (start 203.4 79.305) (end 202.095 79.305) (width 0.6) (layer F.Cu) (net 11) (status 400000))
 (segment (start 201.6 79.8) (end 201.6 81.25) (width 0.6) (layer F.Cu) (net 11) (status 800000))
 (segment (start 202.095 79.305) (end 201.6 79.8) (width 0.6) (layer F.Cu) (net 11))
 (segment (start 201.6 81.25) (end 201.95 81.6) (width 0.6) (layer F.Cu) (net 11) (status C00000))
 (segment (start 202.25 81.3) (end 201.95 81.6) (width 0.6) (layer F.Cu) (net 11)))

